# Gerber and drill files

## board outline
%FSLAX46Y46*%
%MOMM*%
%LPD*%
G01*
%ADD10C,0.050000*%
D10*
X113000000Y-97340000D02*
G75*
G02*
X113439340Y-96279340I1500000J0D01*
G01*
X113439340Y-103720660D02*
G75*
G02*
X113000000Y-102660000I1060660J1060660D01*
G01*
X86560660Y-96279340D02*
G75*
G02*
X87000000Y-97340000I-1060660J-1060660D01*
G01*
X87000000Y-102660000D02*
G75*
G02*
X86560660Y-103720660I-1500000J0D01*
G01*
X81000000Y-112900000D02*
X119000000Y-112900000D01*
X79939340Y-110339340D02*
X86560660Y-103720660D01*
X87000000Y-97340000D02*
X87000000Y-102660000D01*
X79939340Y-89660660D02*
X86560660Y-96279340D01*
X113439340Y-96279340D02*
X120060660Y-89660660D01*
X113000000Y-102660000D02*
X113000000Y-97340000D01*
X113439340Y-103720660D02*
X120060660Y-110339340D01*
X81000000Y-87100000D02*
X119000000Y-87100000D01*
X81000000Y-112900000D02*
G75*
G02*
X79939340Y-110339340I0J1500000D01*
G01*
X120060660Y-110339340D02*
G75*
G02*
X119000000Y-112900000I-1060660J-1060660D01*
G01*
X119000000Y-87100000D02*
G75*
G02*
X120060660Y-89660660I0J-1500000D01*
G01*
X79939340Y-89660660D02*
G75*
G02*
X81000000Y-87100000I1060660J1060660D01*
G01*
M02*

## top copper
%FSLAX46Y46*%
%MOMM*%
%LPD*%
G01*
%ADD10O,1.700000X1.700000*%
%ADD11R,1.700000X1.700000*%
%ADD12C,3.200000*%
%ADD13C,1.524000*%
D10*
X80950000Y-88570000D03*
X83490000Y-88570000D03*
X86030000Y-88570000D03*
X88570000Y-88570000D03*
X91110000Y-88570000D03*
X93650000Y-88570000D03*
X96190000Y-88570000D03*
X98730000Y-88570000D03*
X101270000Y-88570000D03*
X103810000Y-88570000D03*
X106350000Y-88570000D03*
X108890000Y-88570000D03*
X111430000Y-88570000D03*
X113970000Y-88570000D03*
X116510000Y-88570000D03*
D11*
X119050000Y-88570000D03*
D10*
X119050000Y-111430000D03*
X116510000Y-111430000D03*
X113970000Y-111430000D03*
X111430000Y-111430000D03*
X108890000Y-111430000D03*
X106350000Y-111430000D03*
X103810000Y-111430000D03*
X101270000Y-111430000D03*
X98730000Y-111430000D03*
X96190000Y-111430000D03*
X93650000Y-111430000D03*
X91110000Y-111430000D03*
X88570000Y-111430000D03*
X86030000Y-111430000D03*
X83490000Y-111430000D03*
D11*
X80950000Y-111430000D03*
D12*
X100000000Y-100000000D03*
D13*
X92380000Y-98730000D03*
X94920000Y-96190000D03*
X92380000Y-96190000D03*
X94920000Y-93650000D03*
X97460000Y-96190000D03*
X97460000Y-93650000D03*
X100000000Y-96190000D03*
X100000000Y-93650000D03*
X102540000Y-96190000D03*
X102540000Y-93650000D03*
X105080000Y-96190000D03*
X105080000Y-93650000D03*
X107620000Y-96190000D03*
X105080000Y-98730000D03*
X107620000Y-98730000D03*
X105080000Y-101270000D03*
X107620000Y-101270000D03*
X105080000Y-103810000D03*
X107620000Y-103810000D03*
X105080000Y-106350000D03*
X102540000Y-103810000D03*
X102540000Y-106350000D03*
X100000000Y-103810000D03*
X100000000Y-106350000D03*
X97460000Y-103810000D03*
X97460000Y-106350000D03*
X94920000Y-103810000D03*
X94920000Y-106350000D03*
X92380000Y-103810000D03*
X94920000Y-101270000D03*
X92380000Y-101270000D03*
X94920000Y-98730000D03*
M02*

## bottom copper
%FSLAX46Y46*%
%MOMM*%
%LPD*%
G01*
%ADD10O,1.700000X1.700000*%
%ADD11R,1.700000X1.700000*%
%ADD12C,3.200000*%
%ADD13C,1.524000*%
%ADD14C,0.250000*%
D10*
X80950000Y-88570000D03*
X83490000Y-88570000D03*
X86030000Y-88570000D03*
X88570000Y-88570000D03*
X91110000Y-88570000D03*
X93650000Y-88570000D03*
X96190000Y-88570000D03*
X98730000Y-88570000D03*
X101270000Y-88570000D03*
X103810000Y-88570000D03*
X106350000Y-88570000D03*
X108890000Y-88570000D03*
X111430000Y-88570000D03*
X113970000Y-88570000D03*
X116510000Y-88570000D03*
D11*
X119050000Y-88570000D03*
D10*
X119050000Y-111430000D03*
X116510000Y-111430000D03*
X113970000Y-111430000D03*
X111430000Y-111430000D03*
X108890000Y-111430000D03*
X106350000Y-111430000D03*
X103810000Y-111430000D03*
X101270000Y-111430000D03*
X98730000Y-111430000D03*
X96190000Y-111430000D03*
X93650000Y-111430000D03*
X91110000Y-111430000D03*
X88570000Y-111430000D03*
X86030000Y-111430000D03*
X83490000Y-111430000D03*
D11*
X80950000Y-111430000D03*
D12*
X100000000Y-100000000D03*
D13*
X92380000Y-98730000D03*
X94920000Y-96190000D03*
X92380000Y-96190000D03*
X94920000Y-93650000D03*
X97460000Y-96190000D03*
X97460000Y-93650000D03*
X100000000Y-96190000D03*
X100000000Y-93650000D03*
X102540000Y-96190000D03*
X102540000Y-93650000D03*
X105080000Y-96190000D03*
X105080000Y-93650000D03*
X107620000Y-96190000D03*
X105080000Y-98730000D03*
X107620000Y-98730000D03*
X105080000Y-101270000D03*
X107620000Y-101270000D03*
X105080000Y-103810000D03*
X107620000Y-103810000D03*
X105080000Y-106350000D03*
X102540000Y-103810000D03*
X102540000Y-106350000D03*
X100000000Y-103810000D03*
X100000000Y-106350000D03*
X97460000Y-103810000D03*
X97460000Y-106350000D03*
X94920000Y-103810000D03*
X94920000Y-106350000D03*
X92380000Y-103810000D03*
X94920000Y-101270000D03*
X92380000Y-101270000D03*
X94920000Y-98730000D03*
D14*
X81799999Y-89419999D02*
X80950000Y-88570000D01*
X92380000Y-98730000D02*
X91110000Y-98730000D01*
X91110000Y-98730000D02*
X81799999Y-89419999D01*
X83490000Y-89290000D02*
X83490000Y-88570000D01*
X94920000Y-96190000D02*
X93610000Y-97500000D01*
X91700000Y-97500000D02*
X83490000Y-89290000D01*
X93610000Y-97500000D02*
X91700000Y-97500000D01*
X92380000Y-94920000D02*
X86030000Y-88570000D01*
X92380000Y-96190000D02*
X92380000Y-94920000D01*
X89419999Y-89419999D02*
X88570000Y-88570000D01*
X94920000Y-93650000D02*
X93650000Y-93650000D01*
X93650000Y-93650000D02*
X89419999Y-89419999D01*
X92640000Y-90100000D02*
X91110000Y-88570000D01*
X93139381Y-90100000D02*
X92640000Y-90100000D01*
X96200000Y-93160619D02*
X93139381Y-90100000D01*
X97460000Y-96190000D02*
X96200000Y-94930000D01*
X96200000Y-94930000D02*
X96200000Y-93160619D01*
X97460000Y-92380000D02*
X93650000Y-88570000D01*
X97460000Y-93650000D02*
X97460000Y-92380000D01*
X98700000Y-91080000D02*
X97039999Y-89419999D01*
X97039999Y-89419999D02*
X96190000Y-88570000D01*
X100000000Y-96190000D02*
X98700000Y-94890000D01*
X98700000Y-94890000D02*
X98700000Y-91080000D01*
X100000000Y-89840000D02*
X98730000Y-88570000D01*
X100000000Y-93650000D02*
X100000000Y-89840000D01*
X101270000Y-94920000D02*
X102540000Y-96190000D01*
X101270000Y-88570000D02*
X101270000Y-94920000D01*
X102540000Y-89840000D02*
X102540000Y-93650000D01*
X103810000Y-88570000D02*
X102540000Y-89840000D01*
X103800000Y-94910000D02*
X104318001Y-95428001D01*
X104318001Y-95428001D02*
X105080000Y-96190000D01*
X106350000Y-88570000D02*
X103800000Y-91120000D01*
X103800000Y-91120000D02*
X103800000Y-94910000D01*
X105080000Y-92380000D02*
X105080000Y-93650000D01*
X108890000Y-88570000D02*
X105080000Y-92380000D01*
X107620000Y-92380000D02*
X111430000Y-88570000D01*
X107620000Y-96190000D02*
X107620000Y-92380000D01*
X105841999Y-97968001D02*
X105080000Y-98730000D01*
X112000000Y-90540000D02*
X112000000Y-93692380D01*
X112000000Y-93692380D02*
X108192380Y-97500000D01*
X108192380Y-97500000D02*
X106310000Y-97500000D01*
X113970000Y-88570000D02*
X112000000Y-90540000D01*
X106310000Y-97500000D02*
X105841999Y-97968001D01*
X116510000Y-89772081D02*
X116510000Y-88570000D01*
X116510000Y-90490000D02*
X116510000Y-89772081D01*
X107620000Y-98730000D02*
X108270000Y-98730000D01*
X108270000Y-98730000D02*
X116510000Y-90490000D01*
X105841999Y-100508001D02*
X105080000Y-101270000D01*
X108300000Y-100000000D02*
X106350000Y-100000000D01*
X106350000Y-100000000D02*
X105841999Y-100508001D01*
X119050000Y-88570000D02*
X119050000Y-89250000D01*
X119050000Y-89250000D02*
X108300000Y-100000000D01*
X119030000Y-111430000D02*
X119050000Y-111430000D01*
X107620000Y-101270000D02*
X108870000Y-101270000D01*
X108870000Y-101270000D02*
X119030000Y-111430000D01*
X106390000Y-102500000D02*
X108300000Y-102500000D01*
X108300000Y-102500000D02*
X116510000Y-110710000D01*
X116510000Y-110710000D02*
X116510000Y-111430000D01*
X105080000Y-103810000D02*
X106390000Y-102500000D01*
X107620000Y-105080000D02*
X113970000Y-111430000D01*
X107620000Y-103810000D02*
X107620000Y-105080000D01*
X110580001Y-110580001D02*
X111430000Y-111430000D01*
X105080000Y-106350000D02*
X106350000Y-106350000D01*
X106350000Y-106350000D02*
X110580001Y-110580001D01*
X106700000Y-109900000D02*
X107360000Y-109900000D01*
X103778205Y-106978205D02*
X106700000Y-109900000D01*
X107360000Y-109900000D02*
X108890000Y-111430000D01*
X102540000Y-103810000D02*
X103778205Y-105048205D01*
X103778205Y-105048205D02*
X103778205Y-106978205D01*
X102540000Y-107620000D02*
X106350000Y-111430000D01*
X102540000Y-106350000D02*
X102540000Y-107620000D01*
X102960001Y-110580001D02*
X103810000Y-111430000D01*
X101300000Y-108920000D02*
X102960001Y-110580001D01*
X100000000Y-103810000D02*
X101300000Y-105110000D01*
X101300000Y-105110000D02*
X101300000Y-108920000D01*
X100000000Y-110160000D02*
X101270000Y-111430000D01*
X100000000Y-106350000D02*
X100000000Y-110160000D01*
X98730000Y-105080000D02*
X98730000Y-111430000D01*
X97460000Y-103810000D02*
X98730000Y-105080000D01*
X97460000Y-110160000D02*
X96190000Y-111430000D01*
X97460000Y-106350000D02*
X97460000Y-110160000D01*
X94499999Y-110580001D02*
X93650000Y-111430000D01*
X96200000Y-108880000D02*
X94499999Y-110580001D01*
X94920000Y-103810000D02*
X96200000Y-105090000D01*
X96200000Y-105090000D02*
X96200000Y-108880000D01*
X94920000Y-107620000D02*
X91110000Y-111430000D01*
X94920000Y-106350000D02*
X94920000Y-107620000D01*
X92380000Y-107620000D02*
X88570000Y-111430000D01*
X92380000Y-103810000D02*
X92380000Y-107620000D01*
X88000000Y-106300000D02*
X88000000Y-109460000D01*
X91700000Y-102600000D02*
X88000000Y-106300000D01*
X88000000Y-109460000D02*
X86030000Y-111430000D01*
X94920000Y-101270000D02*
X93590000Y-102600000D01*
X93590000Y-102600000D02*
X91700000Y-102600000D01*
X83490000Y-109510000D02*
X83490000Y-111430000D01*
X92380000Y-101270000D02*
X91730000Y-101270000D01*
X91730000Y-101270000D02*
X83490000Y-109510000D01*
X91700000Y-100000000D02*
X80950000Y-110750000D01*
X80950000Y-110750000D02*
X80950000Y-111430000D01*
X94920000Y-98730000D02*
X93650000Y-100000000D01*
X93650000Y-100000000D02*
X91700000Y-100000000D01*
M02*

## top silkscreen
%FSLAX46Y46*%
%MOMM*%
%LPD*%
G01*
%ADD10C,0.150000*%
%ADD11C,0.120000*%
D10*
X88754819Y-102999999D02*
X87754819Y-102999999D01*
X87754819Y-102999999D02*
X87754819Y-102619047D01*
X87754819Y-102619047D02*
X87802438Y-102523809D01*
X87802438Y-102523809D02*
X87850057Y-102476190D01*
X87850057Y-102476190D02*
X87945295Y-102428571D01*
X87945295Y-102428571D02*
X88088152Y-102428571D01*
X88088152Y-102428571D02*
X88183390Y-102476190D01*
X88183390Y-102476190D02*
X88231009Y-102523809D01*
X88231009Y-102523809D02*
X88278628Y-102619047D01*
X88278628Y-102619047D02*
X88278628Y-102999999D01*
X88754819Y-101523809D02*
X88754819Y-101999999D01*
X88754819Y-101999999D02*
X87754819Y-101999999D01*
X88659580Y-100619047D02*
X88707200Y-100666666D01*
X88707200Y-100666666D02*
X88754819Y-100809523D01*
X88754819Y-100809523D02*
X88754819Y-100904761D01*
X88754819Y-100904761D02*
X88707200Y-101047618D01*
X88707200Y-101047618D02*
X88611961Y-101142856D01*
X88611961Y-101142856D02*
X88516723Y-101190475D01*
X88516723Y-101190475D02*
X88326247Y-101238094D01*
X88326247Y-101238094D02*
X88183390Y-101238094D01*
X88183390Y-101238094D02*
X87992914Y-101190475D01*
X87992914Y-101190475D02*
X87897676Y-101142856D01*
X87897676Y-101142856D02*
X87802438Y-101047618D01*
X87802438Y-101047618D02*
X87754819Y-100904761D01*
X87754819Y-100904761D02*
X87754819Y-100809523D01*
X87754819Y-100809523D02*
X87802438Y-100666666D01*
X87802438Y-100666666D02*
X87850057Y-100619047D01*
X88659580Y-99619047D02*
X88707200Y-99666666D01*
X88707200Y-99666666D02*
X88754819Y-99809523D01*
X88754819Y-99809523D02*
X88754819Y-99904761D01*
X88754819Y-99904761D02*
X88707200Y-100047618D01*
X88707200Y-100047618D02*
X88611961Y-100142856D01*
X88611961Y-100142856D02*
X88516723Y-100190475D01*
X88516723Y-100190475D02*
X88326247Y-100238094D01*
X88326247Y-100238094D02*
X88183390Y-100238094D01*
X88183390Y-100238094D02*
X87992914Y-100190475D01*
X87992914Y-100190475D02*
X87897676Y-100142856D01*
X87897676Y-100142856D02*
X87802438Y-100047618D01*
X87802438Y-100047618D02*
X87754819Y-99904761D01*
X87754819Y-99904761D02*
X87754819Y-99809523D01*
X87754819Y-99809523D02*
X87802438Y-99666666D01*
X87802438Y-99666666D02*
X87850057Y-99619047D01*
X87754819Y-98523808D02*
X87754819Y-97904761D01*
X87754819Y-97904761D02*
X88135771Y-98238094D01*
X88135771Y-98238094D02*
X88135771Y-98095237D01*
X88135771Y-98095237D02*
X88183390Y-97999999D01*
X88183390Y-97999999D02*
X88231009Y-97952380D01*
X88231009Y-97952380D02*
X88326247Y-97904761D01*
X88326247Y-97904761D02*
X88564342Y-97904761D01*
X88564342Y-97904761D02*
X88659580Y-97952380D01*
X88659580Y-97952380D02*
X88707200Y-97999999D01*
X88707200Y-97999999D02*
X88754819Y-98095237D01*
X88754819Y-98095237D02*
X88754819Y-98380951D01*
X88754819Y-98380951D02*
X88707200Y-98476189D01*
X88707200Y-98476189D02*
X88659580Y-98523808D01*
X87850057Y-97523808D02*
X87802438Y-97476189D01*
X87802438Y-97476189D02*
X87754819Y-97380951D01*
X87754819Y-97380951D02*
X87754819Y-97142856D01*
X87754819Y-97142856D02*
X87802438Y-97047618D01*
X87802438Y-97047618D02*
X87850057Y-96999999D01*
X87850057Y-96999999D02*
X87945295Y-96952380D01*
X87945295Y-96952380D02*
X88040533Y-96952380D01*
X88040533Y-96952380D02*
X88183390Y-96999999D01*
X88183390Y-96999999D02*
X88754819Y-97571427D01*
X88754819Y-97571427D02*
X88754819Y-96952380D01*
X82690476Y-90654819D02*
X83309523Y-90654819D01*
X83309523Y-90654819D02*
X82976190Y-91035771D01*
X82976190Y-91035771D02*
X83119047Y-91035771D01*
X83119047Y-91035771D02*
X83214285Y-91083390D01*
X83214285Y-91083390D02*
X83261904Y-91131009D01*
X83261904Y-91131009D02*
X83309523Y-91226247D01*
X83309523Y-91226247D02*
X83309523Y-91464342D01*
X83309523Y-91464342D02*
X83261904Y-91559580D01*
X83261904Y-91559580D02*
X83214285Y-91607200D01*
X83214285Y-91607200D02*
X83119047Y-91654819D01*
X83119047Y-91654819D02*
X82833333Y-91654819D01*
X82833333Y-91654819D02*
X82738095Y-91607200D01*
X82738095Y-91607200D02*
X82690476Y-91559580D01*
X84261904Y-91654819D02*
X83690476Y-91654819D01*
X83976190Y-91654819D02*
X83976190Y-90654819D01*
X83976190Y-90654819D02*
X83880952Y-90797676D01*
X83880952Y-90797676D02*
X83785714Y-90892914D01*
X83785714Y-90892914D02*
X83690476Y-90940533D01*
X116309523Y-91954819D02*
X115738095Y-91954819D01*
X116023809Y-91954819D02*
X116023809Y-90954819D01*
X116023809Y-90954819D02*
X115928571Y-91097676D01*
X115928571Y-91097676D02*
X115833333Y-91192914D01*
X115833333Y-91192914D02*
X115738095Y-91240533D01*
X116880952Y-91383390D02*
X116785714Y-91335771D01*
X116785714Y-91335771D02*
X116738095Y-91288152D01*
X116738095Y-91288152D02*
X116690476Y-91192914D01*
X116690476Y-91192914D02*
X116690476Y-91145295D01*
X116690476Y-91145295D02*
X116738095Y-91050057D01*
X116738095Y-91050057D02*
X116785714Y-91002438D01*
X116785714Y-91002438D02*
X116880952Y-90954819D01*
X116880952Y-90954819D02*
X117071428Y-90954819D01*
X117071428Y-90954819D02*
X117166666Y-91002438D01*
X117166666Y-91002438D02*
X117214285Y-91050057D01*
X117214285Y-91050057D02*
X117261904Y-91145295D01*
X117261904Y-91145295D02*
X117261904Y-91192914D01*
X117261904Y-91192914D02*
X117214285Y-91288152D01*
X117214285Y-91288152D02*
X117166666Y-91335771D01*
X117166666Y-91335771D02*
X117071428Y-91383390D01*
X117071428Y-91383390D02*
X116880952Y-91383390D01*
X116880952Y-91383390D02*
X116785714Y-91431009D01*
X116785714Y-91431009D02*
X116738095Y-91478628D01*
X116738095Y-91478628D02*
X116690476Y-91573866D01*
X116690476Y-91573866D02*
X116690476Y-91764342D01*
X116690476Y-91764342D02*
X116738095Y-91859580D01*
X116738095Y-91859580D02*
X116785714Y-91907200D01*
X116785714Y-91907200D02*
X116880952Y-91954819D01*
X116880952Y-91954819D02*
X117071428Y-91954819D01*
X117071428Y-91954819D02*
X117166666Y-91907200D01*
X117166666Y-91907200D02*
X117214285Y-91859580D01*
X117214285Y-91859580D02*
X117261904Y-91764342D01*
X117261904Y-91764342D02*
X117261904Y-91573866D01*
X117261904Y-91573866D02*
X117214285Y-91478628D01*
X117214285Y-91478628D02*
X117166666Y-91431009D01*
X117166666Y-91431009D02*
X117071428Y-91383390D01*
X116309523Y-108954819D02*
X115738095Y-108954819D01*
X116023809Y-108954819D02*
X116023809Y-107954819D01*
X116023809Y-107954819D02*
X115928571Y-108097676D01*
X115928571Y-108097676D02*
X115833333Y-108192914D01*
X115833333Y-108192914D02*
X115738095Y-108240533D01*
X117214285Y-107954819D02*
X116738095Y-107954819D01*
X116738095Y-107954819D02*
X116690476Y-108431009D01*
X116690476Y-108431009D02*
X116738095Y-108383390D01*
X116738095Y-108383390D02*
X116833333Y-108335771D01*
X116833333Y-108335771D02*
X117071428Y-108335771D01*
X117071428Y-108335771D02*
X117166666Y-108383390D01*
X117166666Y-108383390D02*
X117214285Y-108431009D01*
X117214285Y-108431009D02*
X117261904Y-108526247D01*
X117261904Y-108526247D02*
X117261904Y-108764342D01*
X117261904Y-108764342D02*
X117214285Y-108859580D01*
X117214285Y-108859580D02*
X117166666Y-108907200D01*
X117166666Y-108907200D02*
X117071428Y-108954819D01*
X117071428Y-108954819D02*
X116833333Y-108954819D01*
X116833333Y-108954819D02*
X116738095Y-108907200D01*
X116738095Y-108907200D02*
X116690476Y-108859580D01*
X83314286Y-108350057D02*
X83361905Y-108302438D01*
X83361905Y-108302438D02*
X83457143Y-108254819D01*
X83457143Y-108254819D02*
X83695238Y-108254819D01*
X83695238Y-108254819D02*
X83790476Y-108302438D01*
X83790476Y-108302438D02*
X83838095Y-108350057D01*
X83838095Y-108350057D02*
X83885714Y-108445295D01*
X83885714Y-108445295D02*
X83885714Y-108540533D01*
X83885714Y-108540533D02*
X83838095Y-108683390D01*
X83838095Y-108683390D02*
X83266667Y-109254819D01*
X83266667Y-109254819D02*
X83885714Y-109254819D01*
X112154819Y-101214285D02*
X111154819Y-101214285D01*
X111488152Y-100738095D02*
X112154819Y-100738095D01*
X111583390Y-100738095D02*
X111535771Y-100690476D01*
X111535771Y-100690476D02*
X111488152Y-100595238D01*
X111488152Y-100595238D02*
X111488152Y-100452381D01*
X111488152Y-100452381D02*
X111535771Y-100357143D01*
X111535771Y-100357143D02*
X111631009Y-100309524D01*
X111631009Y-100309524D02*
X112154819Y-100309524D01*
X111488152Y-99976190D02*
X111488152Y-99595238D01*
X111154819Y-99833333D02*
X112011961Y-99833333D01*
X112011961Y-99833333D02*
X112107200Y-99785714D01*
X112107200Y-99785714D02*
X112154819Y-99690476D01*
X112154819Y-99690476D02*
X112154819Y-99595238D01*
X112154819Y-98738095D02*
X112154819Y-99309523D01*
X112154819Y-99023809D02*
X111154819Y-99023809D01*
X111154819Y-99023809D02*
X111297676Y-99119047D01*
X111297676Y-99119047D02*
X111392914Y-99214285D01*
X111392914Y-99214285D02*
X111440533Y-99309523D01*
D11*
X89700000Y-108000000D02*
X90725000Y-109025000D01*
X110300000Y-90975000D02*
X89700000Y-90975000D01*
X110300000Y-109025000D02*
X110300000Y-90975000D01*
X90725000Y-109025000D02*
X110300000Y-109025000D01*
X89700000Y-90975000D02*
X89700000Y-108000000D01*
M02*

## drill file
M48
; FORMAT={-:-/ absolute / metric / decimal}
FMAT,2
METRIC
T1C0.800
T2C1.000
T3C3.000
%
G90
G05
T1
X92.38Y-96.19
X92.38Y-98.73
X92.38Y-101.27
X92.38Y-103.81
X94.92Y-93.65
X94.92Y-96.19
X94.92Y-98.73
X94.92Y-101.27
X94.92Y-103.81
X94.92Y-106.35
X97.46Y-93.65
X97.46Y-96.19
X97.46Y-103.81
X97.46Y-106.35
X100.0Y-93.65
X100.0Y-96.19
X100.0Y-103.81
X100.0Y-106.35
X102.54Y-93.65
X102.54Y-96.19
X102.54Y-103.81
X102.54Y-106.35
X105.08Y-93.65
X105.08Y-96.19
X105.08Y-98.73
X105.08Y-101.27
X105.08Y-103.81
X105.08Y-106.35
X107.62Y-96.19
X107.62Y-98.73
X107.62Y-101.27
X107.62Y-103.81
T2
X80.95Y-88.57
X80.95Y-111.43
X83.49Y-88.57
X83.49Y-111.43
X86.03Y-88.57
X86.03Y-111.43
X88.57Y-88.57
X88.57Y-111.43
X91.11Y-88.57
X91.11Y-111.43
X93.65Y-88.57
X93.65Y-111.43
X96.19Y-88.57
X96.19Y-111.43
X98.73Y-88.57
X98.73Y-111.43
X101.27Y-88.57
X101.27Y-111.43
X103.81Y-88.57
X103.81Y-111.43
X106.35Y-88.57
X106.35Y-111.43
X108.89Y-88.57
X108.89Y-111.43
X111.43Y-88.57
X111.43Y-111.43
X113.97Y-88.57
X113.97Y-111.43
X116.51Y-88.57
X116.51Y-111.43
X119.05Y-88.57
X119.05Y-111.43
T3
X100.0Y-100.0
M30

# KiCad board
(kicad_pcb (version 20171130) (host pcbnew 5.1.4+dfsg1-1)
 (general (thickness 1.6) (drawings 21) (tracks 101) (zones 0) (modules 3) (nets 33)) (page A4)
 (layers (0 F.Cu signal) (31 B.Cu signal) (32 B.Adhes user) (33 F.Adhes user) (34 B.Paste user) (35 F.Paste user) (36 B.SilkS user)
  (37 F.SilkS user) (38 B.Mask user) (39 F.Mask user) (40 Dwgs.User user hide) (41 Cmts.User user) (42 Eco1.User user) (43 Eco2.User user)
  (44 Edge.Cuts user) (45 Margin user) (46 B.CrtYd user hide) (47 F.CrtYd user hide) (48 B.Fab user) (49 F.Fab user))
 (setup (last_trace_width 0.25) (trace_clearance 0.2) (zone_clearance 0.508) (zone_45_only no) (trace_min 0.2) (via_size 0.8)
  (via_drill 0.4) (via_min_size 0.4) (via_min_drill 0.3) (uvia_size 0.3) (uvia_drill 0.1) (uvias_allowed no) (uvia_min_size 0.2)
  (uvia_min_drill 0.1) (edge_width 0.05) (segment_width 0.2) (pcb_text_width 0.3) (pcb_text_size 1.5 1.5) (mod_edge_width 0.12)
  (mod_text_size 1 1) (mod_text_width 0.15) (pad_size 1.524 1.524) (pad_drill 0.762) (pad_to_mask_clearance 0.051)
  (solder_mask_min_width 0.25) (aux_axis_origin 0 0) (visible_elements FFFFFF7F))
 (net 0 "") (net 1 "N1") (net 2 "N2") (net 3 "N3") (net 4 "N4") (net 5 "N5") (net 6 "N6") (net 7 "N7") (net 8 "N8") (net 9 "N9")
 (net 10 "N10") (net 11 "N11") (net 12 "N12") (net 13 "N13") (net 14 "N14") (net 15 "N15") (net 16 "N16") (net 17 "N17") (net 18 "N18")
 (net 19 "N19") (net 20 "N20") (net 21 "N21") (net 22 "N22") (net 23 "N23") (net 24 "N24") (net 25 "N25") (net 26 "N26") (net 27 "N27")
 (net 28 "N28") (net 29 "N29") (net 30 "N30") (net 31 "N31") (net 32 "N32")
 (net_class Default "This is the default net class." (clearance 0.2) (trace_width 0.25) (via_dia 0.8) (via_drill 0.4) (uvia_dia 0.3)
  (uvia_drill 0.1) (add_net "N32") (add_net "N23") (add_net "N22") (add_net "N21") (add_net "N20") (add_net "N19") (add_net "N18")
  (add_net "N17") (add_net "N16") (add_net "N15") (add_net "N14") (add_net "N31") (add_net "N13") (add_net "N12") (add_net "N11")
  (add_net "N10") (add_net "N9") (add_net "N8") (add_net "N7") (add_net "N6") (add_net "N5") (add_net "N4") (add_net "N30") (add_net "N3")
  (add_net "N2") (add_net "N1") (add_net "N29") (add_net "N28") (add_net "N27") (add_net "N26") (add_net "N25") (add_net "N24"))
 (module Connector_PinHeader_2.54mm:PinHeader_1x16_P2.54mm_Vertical (layer B.Cu) (at 119.05 88.57 90)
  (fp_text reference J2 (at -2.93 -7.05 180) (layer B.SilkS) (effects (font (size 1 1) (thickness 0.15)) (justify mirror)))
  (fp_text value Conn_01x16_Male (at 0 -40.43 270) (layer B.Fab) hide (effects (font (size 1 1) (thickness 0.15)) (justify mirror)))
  (pad 16 thru_hole oval (at 0 -38.1 90) (size 1.7 1.7) (drill 1) (layers *.Cu *.Mask) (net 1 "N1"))
  (pad 15 thru_hole oval (at 0 -35.56 90) (size 1.7 1.7) (drill 1) (layers *.Cu *.Mask) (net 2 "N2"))
  (pad 14 thru_hole oval (at 0 -33.02 90) (size 1.7 1.7) (drill 1) (layers *.Cu *.Mask) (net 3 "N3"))
  (pad 13 thru_hole oval (at 0 -30.48 90) (size 1.7 1.7) (drill 1) (layers *.Cu *.Mask) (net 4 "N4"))
  (pad 12 thru_hole oval (at 0 -27.94 90) (size 1.7 1.7) (drill 1) (layers *.Cu *.Mask) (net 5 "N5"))
  (pad 11 thru_hole oval (at 0 -25.4 90) (size 1.7 1.7) (drill 1) (layers *.Cu *.Mask) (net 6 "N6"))
  (pad 10 thru_hole oval (at 0 -22.86 90) (size 1.7 1.7) (drill 1) (layers *.Cu *.Mask) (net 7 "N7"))
  (pad 9 thru_hole oval (at 0 -20.32 90) (size 1.7 1.7) (drill 1) (layers *.Cu *.Mask) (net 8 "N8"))
  (pad 8 thru_hole oval (at 0 -17.78 90) (size 1.7 1.7) (drill 1) (layers *.Cu *.Mask) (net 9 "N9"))
  (pad 7 thru_hole oval (at 0 -15.24 90) (size 1.7 1.7) (drill 1) (layers *.Cu *.Mask) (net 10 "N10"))
  (pad 6 thru_hole oval (at 0 -12.7 90) (size 1.7 1.7) (drill 1) (layers *.Cu *.Mask) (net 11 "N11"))
  (pad 5 thru_hole oval (at 0 -10.16 90) (size 1.7 1.7) (drill 1) (layers *.Cu *.Mask) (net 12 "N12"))
  (pad 4 thru_hole oval (at 0 -7.62 90) (size 1.7 1.7) (drill 1) (layers *.Cu *.Mask) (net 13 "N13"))
  (pad 3 thru_hole oval (at 0 -5.08 90) (size 1.7 1.7) (drill 1) (layers *.Cu *.Mask) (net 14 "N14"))
  (pad 2 thru_hole oval (at 0 -2.54 90) (size 1.7 1.7) (drill 1) (layers *.Cu *.Mask) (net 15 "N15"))
  (pad 1 thru_hole rect (at 0 0 90) (size 1.7 1.7) (drill 1) (layers *.Cu *.Mask) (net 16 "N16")))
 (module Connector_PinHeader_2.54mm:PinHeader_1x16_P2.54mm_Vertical (layer B.Cu) (at 80.95 111.43 270)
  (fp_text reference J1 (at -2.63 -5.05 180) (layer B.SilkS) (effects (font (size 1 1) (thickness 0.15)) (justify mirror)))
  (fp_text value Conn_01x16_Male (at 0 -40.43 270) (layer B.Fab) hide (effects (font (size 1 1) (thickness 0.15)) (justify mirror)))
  (pad 16 thru_hole oval (at 0 -38.1 270) (size 1.7 1.7) (drill 1) (layers *.Cu *.Mask) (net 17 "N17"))
  (pad 15 thru_hole oval (at 0 -35.56 270) (size 1.7 1.7) (drill 1) (layers *.Cu *.Mask) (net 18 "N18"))
  (pad 14 thru_hole oval (at 0 -33.02 270) (size 1.7 1.7) (drill 1) (layers *.Cu *.Mask) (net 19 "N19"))
  (pad 13 thru_hole oval (at 0 -30.48 270) (size 1.7 1.7) (drill 1) (layers *.Cu *.Mask) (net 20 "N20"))
  (pad 12 thru_hole oval (at 0 -27.94 270) (size 1.7 1.7) (drill 1) (layers *.Cu *.Mask) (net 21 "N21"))
  (pad 11 thru_hole oval (at 0 -25.4 270) (size 1.7 1.7) (drill 1) (layers *.Cu *.Mask) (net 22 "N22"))
  (pad 10 thru_hole oval (at 0 -22.86 270) (size 1.7 1.7) (drill 1) (layers *.Cu *.Mask) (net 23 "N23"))
  (pad 9 thru_hole oval (at 0 -20.32 270) (size 1.7 1.7) (drill 1) (layers *.Cu *.Mask) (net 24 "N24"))
  (pad 8 thru_hole oval (at 0 -17.78 270) (size 1.7 1.7) (drill 1) (layers *.Cu *.Mask) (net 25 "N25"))
  (pad 7 thru_hole oval (at 0 -15.24 270) (size 1.7 1.7) (drill 1) (layers *.Cu *.Mask) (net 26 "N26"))
  (pad 6 thru_hole oval (at 0 -12.7 270) (size 1.7 1.7) (drill 1) (layers *.Cu *.Mask) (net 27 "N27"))
  (pad 5 thru_hole oval (at 0 -10.16 270) (size 1.7 1.7) (drill 1) (layers *.Cu *.Mask) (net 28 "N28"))
  (pad 4 thru_hole oval (at 0 -7.62 270) (size 1.7 1.7) (drill 1) (layers *.Cu *.Mask) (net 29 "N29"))
  (pad 3 thru_hole oval (at 0 -5.08 270) (size 1.7 1.7) (drill 1) (layers *.Cu *.Mask) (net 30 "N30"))
  (pad 2 thru_hole oval (at 0 -2.54 270) (size 1.7 1.7) (drill 1) (layers *.Cu *.Mask) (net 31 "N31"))
  (pad 1 thru_hole rect (at 0 0 270) (size 1.7 1.7) (drill 1) (layers *.Cu *.Mask) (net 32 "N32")))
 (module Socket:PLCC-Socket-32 (layer F.Cu) (at 100 100 90)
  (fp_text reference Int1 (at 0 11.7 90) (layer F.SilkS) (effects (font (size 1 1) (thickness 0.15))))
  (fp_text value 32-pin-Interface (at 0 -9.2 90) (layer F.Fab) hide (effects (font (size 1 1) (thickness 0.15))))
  (fp_line (start -8 -10.3) (end -9.025 -9.275) (layer F.SilkS) (width 0.12))
  (fp_line (start 9.025 10.3) (end 9.025 -10.3) (layer F.SilkS) (width 0.12))
  (fp_line (start -9.025 10.3) (end 9.025 10.3) (layer F.SilkS) (width 0.12))
  (fp_line (start -9.025 -9.275) (end -9.025 10.3) (layer F.SilkS) (width 0.12))
  (fp_line (start 9.025 -10.3) (end -8 -10.3) (layer F.SilkS) (width 0.12))
  (pad "" np_thru_hole circle (at 0 0 90) (size 3.2 3.2) (drill 3) (layers *.Cu *.Mask))
  (pad 32 thru_hole circle (at 1.27 -7.62 90) (size 1.524 1.524) (drill 0.8) (layers *.Cu *.Mask) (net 1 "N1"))
  (pad 31 thru_hole circle (at 3.81 -5.08 90) (size 1.524 1.524) (drill 0.8) (layers *.Cu *.Mask) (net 2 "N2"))
  (pad 30 thru_hole circle (at 3.81 -7.62 90) (size 1.524 1.524) (drill 0.8) (layers *.Cu *.Mask) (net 3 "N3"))
  (pad 29 thru_hole circle (at 6.35 -5.08 90) (size 1.524 1.524) (drill 0.8) (layers *.Cu *.Mask) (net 4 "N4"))
  (pad 28 thru_hole circle (at 3.81 -2.54 90) (size 1.524 1.524) (drill 0.8) (layers *.Cu *.Mask) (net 5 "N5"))
  (pad 27 thru_hole circle (at 6.35 -2.54 90) (size 1.524 1.524) (drill 0.8) (layers *.Cu *.Mask) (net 6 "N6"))
  (pad 26 thru_hole circle (at 3.81 0 90) (size 1.524 1.524) (drill 0.8) (layers *.Cu *.Mask) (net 7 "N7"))
  (pad 25 thru_hole circle (at 6.35 0 90) (size 1.524 1.524) (drill 0.8) (layers *.Cu *.Mask) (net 8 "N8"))
  (pad 24 thru_hole circle (at 3.81 2.54 90) (size 1.524 1.524) (drill 0.8) (layers *.Cu *.Mask) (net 9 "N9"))
  (pad 23 thru_hole circle (at 6.35 2.54 90) (size 1.524 1.524) (drill 0.8) (layers *.Cu *.Mask) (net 10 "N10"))
  (pad 22 thru_hole circle (at 3.81 5.08 90) (size 1.524 1.524) (drill 0.8) (layers *.Cu *.Mask) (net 11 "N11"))
  (pad 21 thru_hole circle (at 6.35 5.08 90) (size 1.524 1.524) (drill 0.8) (layers *.Cu *.Mask) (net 12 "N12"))
  (pad 20 thru_hole circle (at 3.81 7.62 90) (size 1.524 1.524) (drill 0.8) (layers *.Cu *.Mask) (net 13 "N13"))
  (pad 19 thru_hole circle (at 1.27 5.08 90) (size 1.524 1.524) (drill 0.8) (layers *.Cu *.Mask) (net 14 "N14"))
  (pad 18 thru_hole circle (at 1.27 7.62 90) (size 1.524 1.524) (drill 0.8) (layers *.Cu *.Mask) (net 15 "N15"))
  (pad 17 thru_hole circle (at -1.27 5.08 90) (size 1.524 1.524) (drill 0.8) (layers *.Cu *.Mask) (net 16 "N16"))
  (pad 16 thru_hole circle (at -1.27 7.62 90) (size 1.524 1.524) (drill 0.8) (layers *.Cu *.Mask) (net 17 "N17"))
  (pad 15 thru_hole circle (at -3.81 5.08 90) (size 1.524 1.524) (drill 0.8) (layers *.Cu *.Mask) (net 18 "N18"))
  (pad 14 thru_hole circle (at -3.81 7.62 90) (size 1.524 1.524) (drill 0.8) (layers *.Cu *.Mask) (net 19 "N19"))
  (pad 13 thru_hole circle (at -6.35 5.08 90) (size 1.524 1.524) (drill 0.8) (layers *.Cu *.Mask) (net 20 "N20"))
  (pad 12 thru_hole circle (at -3.81 2.54 90) (size 1.524 1.524) (drill 0.8) (layers *.Cu *.Mask) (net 21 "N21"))
  (pad 11 thru_hole circle (at -6.35 2.54 90) (size 1.524 1.524) (drill 0.8) (layers *.Cu *.Mask) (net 22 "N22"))
  (pad 10 thru_hole circle (at -3.81 0 90) (size 1.524 1.524) (drill 0.8) (layers *.Cu *.Mask) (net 23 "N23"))
  (pad 9 thru_hole circle (at -6.35 0 90) (size 1.524 1.524) (drill 0.8) (layers *.Cu *.Mask) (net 24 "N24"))
  (pad 8 thru_hole circle (at -3.81 -2.54 90) (size 1.524 1.524) (drill 0.8) (layers *.Cu *.Mask) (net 25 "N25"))
  (pad 7 thru_hole circle (at -6.35 -2.54 90) (size 1.524 1.524) (drill 0.8) (layers *.Cu *.Mask) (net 26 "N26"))
  (pad 6 thru_hole circle (at -3.81 -5.08 90) (size 1.524 1.524) (drill 0.8) (layers *.Cu *.Mask) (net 27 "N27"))
  (pad 5 thru_hole circle (at -6.35 -5.08 90) (size 1.524 1.524) (drill 0.8) (layers *.Cu *.Mask) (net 28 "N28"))
  (pad 4 thru_hole circle (at -3.81 -7.62 90) (size 1.524 1.524) (drill 0.8) (layers *.Cu *.Mask) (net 29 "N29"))
  (pad 3 thru_hole circle (at -1.27 -5.08 90) (size 1.524 1.524) (drill 0.8) (layers *.Cu *.Mask) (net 30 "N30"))
  (pad 2 thru_hole circle (at -1.27 -7.62 90) (size 1.524 1.524) (drill 0.8) (layers *.Cu *.Mask) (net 31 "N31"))
  (pad 1 thru_hole circle (at 1.27 -5.08 90) (size 1.524 1.524) (drill 0.8) (layers *.Cu *.Mask) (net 32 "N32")))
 (gr_arc (start 114.5 97.34) (end 113 97.34) (angle 45) (layer Edge.Cuts) (width 0.05))
 (gr_arc (start 114.5 102.66) (end 113 102.66) (angle -45) (layer Edge.Cuts) (width 0.05))
 (gr_arc (start 85.5 97.34) (end 87 97.34) (angle -45) (layer Edge.Cuts) (width 0.05))
 (gr_arc (start 85.5 102.66) (end 87 102.66) (angle 45) (layer Edge.Cuts) (width 0.05))
 (gr_line (start 81 112.9) (end 119 112.9) (layer Edge.Cuts) (width 0.05))
 (gr_line (start 79.93934 110.33934) (end 86.56066 103.72066) (layer Edge.Cuts) (width 0.05))
 (gr_line (start 87 97.34) (end 87 102.66) (layer Edge.Cuts) (width 0.05))
 (gr_line (start 79.93934 89.66066) (end 86.56066 96.27934) (layer Edge.Cuts) (width 0.05))
 (gr_line (start 113.43934 96.27934) (end 120.06066 89.66066) (layer Edge.Cuts) (width 0.05))
 (gr_line (start 113 102.66) (end 113 97.34) (layer Edge.Cuts) (width 0.05))
 (gr_line (start 113.43934 103.72066) (end 120.06066 110.33934) (layer Edge.Cuts) (width 0.05))
 (gr_line (start 81 87.1) (end 119 87.1) (layer Edge.Cuts) (width 0.05))
 (gr_arc (start 81 111.4) (end 81 112.9) (angle 135) (layer Edge.Cuts) (width 0.05))
 (gr_arc (start 119 111.4) (end 119 112.9) (angle -135) (layer Edge.Cuts) (width 0.05))
 (gr_arc (start 119 88.6) (end 119 87.1) (angle 135) (layer Edge.Cuts) (width 0.05))
 (gr_arc (start 81 88.6) (end 81 87.1) (angle -135) (layer Edge.Cuts) (width 0.05))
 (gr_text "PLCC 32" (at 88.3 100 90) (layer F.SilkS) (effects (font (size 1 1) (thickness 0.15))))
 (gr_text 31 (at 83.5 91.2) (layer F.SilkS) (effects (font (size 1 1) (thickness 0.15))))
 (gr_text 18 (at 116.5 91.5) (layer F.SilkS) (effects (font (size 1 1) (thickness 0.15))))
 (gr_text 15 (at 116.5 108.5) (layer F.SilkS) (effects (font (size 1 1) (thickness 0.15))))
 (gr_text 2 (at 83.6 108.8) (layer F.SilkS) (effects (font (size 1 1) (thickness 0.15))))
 (segment (start 81.799999 89.419999) (end 80.95 88.57) (width 0.25) (layer B.Cu) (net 1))
 (segment (start 92.38 98.73) (end 91.11 98.73) (width 0.25) (layer B.Cu) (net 1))
 (segment (start 91.11 98.73) (end 81.799999 89.419999) (width 0.25) (layer B.Cu) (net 1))
 (segment (start 83.49 89.29) (end 83.49 88.57) (width 0.25) (layer B.Cu) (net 2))
 (segment (start 94.92 96.19) (end 93.61 97.5) (width 0.25) (layer B.Cu) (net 2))
 (segment (start 91.7 97.5) (end 83.49 89.29) (width 0.25) (layer B.Cu) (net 2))
 (segment (start 93.61 97.5) (end 91.7 97.5) (width 0.25) (layer B.Cu) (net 2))
 (segment (start 92.38 94.92) (end 86.03 88.57) (width 0.25) (layer B.Cu) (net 3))
 (segment (start 92.38 96.19) (end 92.38 94.92) (width 0.25) (layer B.Cu) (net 3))
 (segment (start 89.419999 89.419999) (end 88.57 88.57) (width 0.25) (layer B.Cu) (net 4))
 (segment (start 94.92 93.65) (end 93.65 93.65) (width 0.25) (layer B.Cu) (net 4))
 (segment (start 93.65 93.65) (end 89.419999 89.419999) (width 0.25) (layer B.Cu) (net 4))
 (segment (start 92.64 90.1) (end 91.11 88.57) (width 0.25) (layer B.Cu) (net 5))
 (segment (start 93.139381 90.1) (end 92.64 90.1) (width 0.25) (layer B.Cu) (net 5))
 (segment (start 96.2 93.160619) (end 93.139381 90.1) (width 0.25) (layer B.Cu) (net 5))
 (segment (start 97.46 96.19) (end 96.2 94.93) (width 0.25) (layer B.Cu) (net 5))
 (segment (start 96.2 94.93) (end 96.2 93.160619) (width 0.25) (layer B.Cu) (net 5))
 (segment (start 97.46 92.38) (end 93.65 88.57) (width 0.25) (layer B.Cu) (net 6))
 (segment (start 97.46 93.65) (end 97.46 92.38) (width 0.25) (layer B.Cu) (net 6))
 (segment (start 98.7 91.08) (end 97.039999 89.419999) (width 0.25) (layer B.Cu) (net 7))
 (segment (start 97.039999 89.419999) (end 96.19 88.57) (width 0.25) (layer B.Cu) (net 7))
 (segment (start 100 96.19) (end 98.7 94.89) (width 0.25) (layer B.Cu) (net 7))
 (segment (start 98.7 94.89) (end 98.7 91.08) (width 0.25) (layer B.Cu) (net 7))
 (segment (start 100 89.84) (end 98.73 88.57) (width 0.25) (layer B.Cu) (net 8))
 (segment (start 100 93.65) (end 100 89.84) (width 0.25) (layer B.Cu) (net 8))
 (segment (start 101.27 94.92) (end 102.54 96.19) (width 0.25) (layer B.Cu) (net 9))
 (segment (start 101.27 88.57) (end 101.27 94.92) (width 0.25) (layer B.Cu) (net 9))
 (segment (start 102.54 89.84) (end 102.54 93.65) (width 0.25) (layer B.Cu) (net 10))
 (segment (start 103.81 88.57) (end 102.54 89.84) (width 0.25) (layer B.Cu) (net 10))
 (segment (start 103.8 94.91) (end 104.318001 95.428001) (width 0.25) (layer B.Cu) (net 11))
 (segment (start 104.318001 95.428001) (end 105.08 96.19) (width 0.25) (layer B.Cu) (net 11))
 (segment (start 106.35 88.57) (end 103.8 91.12) (width 0.25) (layer B.Cu) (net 11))
 (segment (start 103.8 91.12) (end 103.8 94.91) (width 0.25) (layer B.Cu) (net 11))
 (segment (start 105.08 92.38) (end 105.08 93.65) (width 0.25) (layer B.Cu) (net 12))
 (segment (start 108.89 88.57) (end 105.08 92.38) (width 0.25) (layer B.Cu) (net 12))
 (segment (start 107.62 92.38) (end 111.43 88.57) (width 0.25) (layer B.Cu) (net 13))
 (segment (start 107.62 96.19) (end 107.62 92.38) (width 0.25) (layer B.Cu) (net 13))
 (segment (start 105.841999 97.968001) (end 105.08 98.73) (width 0.25) (layer B.Cu) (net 14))
 (segment (start 112 90.54) (end 112 93.69238) (width 0.25) (layer B.Cu) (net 14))
 (segment (start 112 93.69238) (end 108.19238 97.5) (width 0.25) (layer B.Cu) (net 14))
 (segment (start 108.19238 97.5) (end 106.31 97.5) (width 0.25) (layer B.Cu) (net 14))
 (segment (start 113.97 88.57) (end 112 90.54) (width 0.25) (layer B.Cu) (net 14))
 (segment (start 106.31 97.5) (end 105.841999 97.968001) (width 0.25) (layer B.Cu) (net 14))
 (segment (start 116.51 89.772081) (end 116.51 88.57) (width 0.25) (layer B.Cu) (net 15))
 (segment (start 116.51 90.49) (end 116.51 89.772081) (width 0.25) (layer B.Cu) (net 15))
 (segment (start 107.62 98.73) (end 108.27 98.73) (width 0.25) (layer B.Cu) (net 15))
 (segment (start 108.27 98.73) (end 116.51 90.49) (width 0.25) (layer B.Cu) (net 15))
 (segment (start 105.841999 100.508001) (end 105.08 101.27) (width 0.25) (layer B.Cu) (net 16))
 (segment (start 108.3 100) (end 106.35 100) (width 0.25) (layer B.Cu) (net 16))
 (segment (start 106.35 100) (end 105.841999 100.508001) (width 0.25) (layer B.Cu) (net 16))
 (segment (start 119.05 88.57) (end 119.05 89.25) (width 0.25) (layer B.Cu) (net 16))
 (segment (start 119.05 89.25) (end 108.3 100) (width 0.25) (layer B.Cu) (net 16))
 (segment (start 119.03 111.43) (end 119.05 111.43) (width 0.25) (layer B.Cu) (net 17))
 (segment (start 107.62 101.27) (end 108.87 101.27) (width 0.25) (layer B.Cu) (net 17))
 (segment (start 108.87 101.27) (end 119.03 111.43) (width 0.25) (layer B.Cu) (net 17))
 (segment (start 106.39 102.5) (end 108.3 102.5) (width 0.25) (layer B.Cu) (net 18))
 (segment (start 108.3 102.5) (end 116.51 110.71) (width 0.25) (layer B.Cu) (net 18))
 (segment (start 116.51 110.71) (end 116.51 111.43) (width 0.25) (layer B.Cu) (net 18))
 (segment (start 105.08 103.81) (end 106.39 102.5) (width 0.25) (layer B.Cu) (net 18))
 (segment (start 107.62 105.08) (end 113.97 111.43) (width 0.25) (layer B.Cu) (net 19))
 (segment (start 107.62 103.81) (end 107.62 105.08) (width 0.25) (layer B.Cu) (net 19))
 (segment (start 110.580001 110.580001) (end 111.43 111.43) (width 0.25) (layer B.Cu) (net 20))
 (segment (start 105.08 106.35) (end 106.35 106.35) (width 0.25) (layer B.Cu) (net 20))
 (segment (start 106.35 106.35) (end 110.580001 110.580001) (width 0.25) (layer B.Cu) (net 20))
 (segment (start 106.7 109.9) (end 107.36 109.9) (width 0.25) (layer B.Cu) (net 21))
 (segment (start 103.778205 106.978205) (end 106.7 109.9) (width 0.25) (layer B.Cu) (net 21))
 (segment (start 107.36 109.9) (end 108.89 111.43) (width 0.25) (layer B.Cu) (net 21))
 (segment (start 102.54 103.81) (end 103.778205 105.048205) (width 0.25) (layer B.Cu) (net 21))
 (segment (start 103.778205 105.048205) (end 103.778205 106.978205) (width 0.25) (layer B.Cu) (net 21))
 (segment (start 102.54 107.62) (end 106.35 111.43) (width 0.25) (layer B.Cu) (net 22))
 (segment (start 102.54 106.35) (end 102.54 107.62) (width 0.25) (layer B.Cu) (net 22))
 (segment (start 102.960001 110.580001) (end 103.81 111.43) (width 0.25) (layer B.Cu) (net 23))
 (segment (start 101.3 108.92) (end 102.960001 110.580001) (width 0.25) (layer B.Cu) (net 23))
 (segment (start 100 103.81) (end 101.3 105.11) (width 0.25) (layer B.Cu) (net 23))
 (segment (start 101.3 105.11) (end 101.3 108.92) (width 0.25) (layer B.Cu) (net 23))
 (segment (start 100 110.16) (end 101.27 111.43) (width 0.25) (layer B.Cu) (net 24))
 (segment (start 100 106.35) (end 100 110.16) (width 0.25) (layer B.Cu) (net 24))
 (segment (start 98.73 105.08) (end 98.73 111.43) (width 0.25) (layer B.Cu) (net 25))
 (segment (start 97.46 103.81) (end 98.73 105.08) (width 0.25) (layer B.Cu) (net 25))
 (segment (start 97.46 110.16) (end 96.19 111.43) (width 0.25) (layer B.Cu) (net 26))
 (segment (start 97.46 106.35) (end 97.46 110.16) (width 0.25) (layer B.Cu) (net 26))
 (segment (start 94.499999 110.580001) (end 93.65 111.43) (width 0.25) (layer B.Cu) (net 27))
 (segment (start 96.2 108.88) (end 94.499999 110.580001) (width 0.25) (layer B.Cu) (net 27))
 (segment (start 94.92 103.81) (end 96.2 105.09) (width 0.25) (layer B.Cu) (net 27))
 (segment (start 96.2 105.09) (end 96.2 108.88) (width 0.25) (layer B.Cu) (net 27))
 (segment (start 94.92 107.62) (end 91.11 111.43) (width 0.25) (layer B.Cu) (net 28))
 (segment (start 94.92 106.35) (end 94.92 107.62) (width 0.25) (layer B.Cu) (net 28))
 (segment (start 92.38 107.62) (end 88.57 111.43) (width 0.25) (layer B.Cu) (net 29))
 (segment (start 92.38 103.81) (end 92.38 107.62) (width 0.25) (layer B.Cu) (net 29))
 (segment (start 88 106.3) (end 88 109.46) (width 0.25) (layer B.Cu) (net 30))
 (segment (start 91.7 102.6) (end 88 106.3) (width 0.25) (layer B.Cu) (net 30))
 (segment (start 88 109.46) (end 86.03 111.43) (width 0.25) (layer B.Cu) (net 30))
 (segment (start 94.92 101.27) (end 93.59 102.6) (width 0.25) (layer B.Cu) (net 30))
 (segment (start 93.59 102.6) (end 91.7 102.6) (width 0.25) (layer B.Cu) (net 30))
 (segment (start 83.49 109.51) (end 83.49 111.43) (width 0.25) (layer B.Cu) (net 31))
 (segment (start 92.38 101.27) (end 91.73 101.27) (width 0.25) (layer B.Cu) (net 31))
 (segment (start 91.73 101.27) (end 83.49 109.51) (width 0.25) (layer B.Cu) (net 31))
 (segment (start 91.7 100) (end 80.95 110.75) (width 0.25) (layer B.Cu) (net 32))
 (segment (start 80.95 110.75) (end 80.95 111.43) (width 0.25) (layer B.Cu) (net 32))
 (segment (start 94.92 98.73) (end 93.65 100) (width 0.25) (layer B.Cu) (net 32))
 (segment (start 93.65 100) (end 91.7 100) (width 0.25) (layer B.Cu) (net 32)))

